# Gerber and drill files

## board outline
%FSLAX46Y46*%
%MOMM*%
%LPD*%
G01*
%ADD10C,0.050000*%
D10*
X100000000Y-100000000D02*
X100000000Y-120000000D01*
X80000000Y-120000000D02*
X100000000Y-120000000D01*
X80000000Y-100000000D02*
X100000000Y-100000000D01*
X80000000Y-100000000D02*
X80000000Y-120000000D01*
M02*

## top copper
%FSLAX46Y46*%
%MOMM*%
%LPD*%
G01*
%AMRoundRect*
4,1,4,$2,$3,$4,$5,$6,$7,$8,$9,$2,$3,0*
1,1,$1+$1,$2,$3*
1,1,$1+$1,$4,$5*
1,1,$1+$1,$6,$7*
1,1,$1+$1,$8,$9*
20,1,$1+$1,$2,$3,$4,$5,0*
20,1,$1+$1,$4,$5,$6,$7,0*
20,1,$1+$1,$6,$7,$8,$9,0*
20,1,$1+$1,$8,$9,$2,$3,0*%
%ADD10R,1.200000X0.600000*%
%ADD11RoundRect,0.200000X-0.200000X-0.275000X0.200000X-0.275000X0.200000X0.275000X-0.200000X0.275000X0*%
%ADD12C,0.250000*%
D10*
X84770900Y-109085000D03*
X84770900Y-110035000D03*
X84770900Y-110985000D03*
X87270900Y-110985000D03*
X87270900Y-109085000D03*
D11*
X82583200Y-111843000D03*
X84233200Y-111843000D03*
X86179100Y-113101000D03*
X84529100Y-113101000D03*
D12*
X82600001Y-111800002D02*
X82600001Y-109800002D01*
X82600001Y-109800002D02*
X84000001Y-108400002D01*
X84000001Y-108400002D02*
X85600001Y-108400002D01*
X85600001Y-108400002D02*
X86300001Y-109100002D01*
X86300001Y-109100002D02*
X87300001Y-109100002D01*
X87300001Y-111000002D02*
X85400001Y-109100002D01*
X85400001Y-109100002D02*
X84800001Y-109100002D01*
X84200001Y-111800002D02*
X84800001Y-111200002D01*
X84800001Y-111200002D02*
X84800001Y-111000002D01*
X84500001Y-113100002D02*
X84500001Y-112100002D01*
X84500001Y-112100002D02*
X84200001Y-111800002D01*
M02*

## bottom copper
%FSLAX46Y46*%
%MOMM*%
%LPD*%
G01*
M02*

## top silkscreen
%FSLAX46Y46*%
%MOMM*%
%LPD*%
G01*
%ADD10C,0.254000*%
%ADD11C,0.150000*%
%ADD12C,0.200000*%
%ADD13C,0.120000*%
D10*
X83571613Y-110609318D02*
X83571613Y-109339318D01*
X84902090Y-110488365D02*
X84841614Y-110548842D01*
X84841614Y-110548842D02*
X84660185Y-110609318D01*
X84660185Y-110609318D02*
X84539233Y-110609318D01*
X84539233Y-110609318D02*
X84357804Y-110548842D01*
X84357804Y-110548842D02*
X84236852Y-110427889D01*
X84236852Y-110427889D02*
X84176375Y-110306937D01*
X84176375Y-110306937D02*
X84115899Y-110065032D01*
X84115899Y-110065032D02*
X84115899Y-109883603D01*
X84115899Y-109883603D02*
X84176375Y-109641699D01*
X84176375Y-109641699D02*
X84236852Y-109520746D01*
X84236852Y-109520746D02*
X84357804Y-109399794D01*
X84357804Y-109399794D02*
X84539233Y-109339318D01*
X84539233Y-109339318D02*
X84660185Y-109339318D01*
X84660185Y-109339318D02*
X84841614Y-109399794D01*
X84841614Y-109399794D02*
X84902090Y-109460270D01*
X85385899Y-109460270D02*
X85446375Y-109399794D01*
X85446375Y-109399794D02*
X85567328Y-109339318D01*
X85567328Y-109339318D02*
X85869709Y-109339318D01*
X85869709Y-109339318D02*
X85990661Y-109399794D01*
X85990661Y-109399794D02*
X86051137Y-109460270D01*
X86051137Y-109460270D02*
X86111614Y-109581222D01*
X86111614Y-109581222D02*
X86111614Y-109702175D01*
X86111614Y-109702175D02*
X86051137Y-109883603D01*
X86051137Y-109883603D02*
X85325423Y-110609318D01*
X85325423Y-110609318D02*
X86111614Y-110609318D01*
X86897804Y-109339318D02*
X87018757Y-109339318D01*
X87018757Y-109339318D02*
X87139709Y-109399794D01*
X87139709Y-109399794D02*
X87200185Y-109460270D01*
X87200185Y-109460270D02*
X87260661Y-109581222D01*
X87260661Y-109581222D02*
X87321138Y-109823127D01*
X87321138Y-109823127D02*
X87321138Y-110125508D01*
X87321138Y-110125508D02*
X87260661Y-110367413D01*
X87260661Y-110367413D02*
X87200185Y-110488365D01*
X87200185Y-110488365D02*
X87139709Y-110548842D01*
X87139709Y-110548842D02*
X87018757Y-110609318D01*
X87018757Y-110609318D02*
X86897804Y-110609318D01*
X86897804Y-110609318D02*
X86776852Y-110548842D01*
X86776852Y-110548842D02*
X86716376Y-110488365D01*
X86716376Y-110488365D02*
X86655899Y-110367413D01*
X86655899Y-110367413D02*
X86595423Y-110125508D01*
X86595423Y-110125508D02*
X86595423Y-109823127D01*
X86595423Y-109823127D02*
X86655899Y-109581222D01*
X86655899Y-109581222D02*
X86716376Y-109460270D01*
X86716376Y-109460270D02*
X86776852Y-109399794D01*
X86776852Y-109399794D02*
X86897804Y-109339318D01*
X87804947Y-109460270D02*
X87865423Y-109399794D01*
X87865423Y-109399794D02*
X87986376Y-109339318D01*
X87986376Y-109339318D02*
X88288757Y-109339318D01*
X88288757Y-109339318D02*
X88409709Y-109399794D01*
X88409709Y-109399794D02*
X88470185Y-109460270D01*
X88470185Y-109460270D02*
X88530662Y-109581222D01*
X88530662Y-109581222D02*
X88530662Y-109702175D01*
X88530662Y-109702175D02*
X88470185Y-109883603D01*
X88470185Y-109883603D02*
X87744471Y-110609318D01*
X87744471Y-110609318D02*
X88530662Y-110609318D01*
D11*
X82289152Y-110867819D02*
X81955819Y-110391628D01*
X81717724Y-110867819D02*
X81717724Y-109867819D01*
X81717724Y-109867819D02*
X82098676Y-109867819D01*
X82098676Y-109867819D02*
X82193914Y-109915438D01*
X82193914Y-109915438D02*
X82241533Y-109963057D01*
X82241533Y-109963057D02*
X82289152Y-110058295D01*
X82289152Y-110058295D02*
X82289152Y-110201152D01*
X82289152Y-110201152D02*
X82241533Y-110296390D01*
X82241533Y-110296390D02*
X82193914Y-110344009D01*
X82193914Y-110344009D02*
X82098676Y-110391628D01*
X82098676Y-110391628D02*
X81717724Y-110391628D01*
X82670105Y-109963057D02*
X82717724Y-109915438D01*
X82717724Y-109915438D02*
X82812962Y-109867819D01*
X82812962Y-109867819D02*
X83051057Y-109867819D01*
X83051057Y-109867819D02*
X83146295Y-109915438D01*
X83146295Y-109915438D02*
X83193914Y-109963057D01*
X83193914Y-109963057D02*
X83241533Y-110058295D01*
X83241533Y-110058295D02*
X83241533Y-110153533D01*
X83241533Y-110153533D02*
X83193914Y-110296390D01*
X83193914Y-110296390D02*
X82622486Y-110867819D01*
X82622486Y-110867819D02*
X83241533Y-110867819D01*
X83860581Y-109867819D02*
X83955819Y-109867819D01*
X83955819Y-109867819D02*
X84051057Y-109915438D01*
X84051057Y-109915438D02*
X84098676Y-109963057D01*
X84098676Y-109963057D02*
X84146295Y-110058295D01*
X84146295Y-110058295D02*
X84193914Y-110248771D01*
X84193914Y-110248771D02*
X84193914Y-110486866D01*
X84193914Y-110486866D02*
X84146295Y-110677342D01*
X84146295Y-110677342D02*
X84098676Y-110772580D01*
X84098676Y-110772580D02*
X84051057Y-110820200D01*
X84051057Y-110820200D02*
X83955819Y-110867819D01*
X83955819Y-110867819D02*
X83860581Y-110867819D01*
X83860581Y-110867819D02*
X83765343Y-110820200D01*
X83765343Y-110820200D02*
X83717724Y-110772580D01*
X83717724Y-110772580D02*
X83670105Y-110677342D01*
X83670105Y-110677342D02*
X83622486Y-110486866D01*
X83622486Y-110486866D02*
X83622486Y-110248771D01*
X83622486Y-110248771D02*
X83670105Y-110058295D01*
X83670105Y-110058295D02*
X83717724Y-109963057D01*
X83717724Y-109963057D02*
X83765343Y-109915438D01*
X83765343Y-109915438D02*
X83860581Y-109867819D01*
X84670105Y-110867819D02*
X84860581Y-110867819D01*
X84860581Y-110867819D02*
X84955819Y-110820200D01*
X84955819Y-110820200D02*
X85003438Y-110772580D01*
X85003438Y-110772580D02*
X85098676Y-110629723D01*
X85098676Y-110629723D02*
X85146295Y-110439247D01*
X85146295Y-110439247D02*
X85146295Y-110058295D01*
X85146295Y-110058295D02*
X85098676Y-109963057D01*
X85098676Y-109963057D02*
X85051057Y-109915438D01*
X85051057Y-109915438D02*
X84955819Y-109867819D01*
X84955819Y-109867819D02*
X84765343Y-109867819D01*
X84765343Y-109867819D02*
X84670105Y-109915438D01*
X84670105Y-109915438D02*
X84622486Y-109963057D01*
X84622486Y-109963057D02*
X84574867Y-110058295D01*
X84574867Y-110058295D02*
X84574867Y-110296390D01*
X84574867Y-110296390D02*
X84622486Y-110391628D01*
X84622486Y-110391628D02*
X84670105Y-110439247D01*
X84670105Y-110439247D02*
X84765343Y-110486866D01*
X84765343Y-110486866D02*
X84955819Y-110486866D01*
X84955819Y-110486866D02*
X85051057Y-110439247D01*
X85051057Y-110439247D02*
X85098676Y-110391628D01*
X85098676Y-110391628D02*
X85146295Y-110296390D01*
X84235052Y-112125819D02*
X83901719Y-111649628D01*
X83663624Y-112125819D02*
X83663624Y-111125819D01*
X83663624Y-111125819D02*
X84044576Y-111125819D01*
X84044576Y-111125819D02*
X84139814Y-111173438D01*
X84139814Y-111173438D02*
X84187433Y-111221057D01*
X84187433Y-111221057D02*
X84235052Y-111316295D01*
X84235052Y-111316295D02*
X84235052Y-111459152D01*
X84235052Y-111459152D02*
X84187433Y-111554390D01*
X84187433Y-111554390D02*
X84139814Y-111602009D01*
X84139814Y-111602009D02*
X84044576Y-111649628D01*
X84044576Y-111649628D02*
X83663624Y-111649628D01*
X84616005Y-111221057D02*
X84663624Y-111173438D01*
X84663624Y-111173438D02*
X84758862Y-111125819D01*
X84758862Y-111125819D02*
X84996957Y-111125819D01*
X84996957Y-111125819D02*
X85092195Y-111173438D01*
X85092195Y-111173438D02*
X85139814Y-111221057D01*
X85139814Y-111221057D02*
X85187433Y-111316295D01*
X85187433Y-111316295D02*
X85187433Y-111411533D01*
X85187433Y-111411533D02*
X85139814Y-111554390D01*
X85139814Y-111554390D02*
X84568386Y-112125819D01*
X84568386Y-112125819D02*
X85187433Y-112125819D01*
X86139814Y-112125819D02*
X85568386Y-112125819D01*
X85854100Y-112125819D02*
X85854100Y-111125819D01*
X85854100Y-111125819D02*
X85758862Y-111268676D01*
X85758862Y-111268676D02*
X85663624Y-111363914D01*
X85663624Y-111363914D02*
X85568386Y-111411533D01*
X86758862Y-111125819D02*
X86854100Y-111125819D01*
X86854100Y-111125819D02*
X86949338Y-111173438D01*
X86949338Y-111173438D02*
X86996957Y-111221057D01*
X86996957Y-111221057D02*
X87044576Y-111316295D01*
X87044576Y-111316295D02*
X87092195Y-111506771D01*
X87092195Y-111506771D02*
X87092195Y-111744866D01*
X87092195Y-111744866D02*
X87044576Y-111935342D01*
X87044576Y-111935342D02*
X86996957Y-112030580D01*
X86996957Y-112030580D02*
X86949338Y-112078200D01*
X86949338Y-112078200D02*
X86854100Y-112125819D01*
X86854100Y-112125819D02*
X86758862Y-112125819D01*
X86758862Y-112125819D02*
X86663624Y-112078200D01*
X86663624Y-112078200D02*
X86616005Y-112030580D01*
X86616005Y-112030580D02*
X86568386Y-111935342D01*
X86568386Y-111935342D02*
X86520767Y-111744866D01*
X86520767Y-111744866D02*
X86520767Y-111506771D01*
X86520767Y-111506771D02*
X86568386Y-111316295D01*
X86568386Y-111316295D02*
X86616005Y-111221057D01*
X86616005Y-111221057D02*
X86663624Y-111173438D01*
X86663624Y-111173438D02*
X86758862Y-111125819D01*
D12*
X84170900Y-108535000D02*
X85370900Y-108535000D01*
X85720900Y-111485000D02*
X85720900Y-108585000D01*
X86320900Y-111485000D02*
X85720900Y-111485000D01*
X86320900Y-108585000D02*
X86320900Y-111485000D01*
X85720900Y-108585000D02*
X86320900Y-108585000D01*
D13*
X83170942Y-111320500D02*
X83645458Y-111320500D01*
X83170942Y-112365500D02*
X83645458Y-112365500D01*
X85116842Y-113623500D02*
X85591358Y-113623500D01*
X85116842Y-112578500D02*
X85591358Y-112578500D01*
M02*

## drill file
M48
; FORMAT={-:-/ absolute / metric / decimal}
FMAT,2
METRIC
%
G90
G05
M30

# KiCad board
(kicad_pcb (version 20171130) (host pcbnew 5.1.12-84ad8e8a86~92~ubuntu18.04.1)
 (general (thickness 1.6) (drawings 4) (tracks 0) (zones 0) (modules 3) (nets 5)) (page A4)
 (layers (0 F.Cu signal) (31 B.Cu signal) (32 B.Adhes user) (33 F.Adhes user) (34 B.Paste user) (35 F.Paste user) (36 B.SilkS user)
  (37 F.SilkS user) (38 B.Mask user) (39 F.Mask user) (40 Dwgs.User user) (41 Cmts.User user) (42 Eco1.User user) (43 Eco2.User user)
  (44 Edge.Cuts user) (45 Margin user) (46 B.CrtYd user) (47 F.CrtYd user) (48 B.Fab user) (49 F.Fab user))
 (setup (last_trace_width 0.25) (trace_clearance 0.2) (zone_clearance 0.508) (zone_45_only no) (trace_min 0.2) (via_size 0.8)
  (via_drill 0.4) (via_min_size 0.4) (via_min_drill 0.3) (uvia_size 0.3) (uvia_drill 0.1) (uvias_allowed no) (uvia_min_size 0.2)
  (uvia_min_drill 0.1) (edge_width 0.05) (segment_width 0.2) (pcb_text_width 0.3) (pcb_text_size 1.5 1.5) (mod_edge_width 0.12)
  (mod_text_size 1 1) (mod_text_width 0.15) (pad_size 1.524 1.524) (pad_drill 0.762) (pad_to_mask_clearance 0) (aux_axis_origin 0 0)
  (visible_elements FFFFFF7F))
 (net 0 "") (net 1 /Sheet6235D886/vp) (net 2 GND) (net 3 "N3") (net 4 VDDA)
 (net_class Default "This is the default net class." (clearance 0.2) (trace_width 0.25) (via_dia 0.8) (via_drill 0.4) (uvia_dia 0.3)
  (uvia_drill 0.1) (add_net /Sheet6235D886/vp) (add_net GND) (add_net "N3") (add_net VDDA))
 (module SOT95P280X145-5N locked (layer F.Cu) (at 86.020900 110.035000)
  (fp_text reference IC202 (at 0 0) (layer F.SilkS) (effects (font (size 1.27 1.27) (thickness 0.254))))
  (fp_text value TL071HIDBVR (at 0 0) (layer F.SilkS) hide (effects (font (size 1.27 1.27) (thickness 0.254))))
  (fp_line (start -1.85 -1.5) (end -0.65 -1.5) (layer F.SilkS) (width 0.2))
  (fp_line (start -0.3 1.45) (end -0.3 -1.45) (layer F.SilkS) (width 0.2))
  (fp_line (start 0.3 1.45) (end -0.3 1.45) (layer F.SilkS) (width 0.2))
  (fp_line (start 0.3 -1.45) (end 0.3 1.45) (layer F.SilkS) (width 0.2))
  (fp_line (start -0.3 -1.45) (end 0.3 -1.45) (layer F.SilkS) (width 0.2))
  (pad 1 smd rect (at -1.25 -0.95 90.000000) (size 0.6 1.2) (layers F.Cu F.Mask F.Paste) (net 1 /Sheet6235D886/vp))
  (pad 2 smd rect (at -1.25 0 90.000000) (size 0.6 1.2) (layers F.Cu F.Mask F.Paste) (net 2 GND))
  (pad 3 smd rect (at -1.25 0.95 90.000000) (size 0.6 1.2) (layers F.Cu F.Mask F.Paste) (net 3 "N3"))
  (pad 4 smd rect (at 1.25 0.95 90.000000) (size 0.6 1.2) (layers F.Cu F.Mask F.Paste) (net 1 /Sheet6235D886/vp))
  (pad 5 smd rect (at 1.25 -0.95 90.000000) (size 0.6 1.2) (layers F.Cu F.Mask F.Paste) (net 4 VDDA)))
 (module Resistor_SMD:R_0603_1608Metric (layer F.Cu) (at 83.408200 111.843000)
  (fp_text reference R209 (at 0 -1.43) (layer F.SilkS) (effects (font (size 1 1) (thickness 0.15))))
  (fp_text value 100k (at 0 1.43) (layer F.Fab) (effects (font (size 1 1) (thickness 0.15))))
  (fp_line (start -0.237258 -0.5225) (end 0.237258 -0.5225) (layer F.SilkS) (width 0.12))
  (fp_line (start -0.237258 0.5225) (end 0.237258 0.5225) (layer F.SilkS) (width 0.12))
  (pad 1 smd roundrect (at -0.825 0) (size 0.8 0.95) (layers F.Cu F.Mask F.Paste) (roundrect_rratio 0.25) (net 4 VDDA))
  (pad 2 smd roundrect (at 0.825 0) (size 0.8 0.95) (layers F.Cu F.Mask F.Paste) (roundrect_rratio 0.25) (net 3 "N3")))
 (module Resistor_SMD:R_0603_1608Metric (layer F.Cu) (at 85.354100 113.101000)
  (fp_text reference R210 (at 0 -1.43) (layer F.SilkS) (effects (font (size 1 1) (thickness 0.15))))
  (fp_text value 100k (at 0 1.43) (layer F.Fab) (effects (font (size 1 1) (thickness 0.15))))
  (fp_line (start -0.237258 0.5225) (end 0.237258 0.5225) (layer F.SilkS) (width 0.12))
  (fp_line (start -0.237258 -0.5225) (end 0.237258 -0.5225) (layer F.SilkS) (width 0.12))
  (pad 2 smd roundrect (at 0.825 0) (size 0.8 0.95) (layers F.Cu F.Mask F.Paste) (roundrect_rratio 0.25) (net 2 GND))
  (pad 1 smd roundrect (at -0.825 0) (size 0.8 0.95) (layers F.Cu F.Mask F.Paste) (roundrect_rratio 0.25) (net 3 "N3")))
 (gr_line (start 100 100) (end 100 120) (layer Edge.Cuts) (width 0.05))
 (gr_line (start 80 120) (end 100 120) (layer Edge.Cuts) (width 0.05))
 (gr_line (start 80 100) (end 100 100) (layer Edge.Cuts) (width 0.05))
 (gr_line (start 80 100) (end 80 120) (layer Edge.Cuts) (width 0.05))
 (segment (start 82.600001 111.800002) (end 82.600001 109.800002) (width 0.250000) (layer F.Cu) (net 4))
 (segment (start 82.600001 109.800002) (end 84.000001 108.400002) (width 0.250000) (layer F.Cu) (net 4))
 (segment (start 84.000001 108.400002) (end 85.600001 108.400002) (width 0.250000) (layer F.Cu) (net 4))
 (segment (start 85.600001 108.400002) (end 86.300001 109.100002) (width 0.250000) (layer F.Cu) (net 4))
 (segment (start 86.300001 109.100002) (end 87.300001 109.100002) (width 0.250000) (layer F.Cu) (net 4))
 (segment (start 87.300001 111.000002) (end 85.400001 109.100002) (width 0.250000) (layer F.Cu) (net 1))
 (segment (start 85.400001 109.100002) (end 84.800001 109.100002) (width 0.250000) (layer F.Cu) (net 1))
 (segment (start 84.200001 111.800002) (end 84.800001 111.200002) (width 0.250000) (layer F.Cu) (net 3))
 (segment (start 84.800001 111.200002) (end 84.800001 111.000002) (width 0.250000) (layer F.Cu) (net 3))
 (segment (start 84.500001 113.100002) (end 84.500001 112.100002) (width 0.250000) (layer F.Cu) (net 3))
 (segment (start 84.500001 112.100002) (end 84.200001 111.800002) (width 0.250000) (layer F.Cu) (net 3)))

